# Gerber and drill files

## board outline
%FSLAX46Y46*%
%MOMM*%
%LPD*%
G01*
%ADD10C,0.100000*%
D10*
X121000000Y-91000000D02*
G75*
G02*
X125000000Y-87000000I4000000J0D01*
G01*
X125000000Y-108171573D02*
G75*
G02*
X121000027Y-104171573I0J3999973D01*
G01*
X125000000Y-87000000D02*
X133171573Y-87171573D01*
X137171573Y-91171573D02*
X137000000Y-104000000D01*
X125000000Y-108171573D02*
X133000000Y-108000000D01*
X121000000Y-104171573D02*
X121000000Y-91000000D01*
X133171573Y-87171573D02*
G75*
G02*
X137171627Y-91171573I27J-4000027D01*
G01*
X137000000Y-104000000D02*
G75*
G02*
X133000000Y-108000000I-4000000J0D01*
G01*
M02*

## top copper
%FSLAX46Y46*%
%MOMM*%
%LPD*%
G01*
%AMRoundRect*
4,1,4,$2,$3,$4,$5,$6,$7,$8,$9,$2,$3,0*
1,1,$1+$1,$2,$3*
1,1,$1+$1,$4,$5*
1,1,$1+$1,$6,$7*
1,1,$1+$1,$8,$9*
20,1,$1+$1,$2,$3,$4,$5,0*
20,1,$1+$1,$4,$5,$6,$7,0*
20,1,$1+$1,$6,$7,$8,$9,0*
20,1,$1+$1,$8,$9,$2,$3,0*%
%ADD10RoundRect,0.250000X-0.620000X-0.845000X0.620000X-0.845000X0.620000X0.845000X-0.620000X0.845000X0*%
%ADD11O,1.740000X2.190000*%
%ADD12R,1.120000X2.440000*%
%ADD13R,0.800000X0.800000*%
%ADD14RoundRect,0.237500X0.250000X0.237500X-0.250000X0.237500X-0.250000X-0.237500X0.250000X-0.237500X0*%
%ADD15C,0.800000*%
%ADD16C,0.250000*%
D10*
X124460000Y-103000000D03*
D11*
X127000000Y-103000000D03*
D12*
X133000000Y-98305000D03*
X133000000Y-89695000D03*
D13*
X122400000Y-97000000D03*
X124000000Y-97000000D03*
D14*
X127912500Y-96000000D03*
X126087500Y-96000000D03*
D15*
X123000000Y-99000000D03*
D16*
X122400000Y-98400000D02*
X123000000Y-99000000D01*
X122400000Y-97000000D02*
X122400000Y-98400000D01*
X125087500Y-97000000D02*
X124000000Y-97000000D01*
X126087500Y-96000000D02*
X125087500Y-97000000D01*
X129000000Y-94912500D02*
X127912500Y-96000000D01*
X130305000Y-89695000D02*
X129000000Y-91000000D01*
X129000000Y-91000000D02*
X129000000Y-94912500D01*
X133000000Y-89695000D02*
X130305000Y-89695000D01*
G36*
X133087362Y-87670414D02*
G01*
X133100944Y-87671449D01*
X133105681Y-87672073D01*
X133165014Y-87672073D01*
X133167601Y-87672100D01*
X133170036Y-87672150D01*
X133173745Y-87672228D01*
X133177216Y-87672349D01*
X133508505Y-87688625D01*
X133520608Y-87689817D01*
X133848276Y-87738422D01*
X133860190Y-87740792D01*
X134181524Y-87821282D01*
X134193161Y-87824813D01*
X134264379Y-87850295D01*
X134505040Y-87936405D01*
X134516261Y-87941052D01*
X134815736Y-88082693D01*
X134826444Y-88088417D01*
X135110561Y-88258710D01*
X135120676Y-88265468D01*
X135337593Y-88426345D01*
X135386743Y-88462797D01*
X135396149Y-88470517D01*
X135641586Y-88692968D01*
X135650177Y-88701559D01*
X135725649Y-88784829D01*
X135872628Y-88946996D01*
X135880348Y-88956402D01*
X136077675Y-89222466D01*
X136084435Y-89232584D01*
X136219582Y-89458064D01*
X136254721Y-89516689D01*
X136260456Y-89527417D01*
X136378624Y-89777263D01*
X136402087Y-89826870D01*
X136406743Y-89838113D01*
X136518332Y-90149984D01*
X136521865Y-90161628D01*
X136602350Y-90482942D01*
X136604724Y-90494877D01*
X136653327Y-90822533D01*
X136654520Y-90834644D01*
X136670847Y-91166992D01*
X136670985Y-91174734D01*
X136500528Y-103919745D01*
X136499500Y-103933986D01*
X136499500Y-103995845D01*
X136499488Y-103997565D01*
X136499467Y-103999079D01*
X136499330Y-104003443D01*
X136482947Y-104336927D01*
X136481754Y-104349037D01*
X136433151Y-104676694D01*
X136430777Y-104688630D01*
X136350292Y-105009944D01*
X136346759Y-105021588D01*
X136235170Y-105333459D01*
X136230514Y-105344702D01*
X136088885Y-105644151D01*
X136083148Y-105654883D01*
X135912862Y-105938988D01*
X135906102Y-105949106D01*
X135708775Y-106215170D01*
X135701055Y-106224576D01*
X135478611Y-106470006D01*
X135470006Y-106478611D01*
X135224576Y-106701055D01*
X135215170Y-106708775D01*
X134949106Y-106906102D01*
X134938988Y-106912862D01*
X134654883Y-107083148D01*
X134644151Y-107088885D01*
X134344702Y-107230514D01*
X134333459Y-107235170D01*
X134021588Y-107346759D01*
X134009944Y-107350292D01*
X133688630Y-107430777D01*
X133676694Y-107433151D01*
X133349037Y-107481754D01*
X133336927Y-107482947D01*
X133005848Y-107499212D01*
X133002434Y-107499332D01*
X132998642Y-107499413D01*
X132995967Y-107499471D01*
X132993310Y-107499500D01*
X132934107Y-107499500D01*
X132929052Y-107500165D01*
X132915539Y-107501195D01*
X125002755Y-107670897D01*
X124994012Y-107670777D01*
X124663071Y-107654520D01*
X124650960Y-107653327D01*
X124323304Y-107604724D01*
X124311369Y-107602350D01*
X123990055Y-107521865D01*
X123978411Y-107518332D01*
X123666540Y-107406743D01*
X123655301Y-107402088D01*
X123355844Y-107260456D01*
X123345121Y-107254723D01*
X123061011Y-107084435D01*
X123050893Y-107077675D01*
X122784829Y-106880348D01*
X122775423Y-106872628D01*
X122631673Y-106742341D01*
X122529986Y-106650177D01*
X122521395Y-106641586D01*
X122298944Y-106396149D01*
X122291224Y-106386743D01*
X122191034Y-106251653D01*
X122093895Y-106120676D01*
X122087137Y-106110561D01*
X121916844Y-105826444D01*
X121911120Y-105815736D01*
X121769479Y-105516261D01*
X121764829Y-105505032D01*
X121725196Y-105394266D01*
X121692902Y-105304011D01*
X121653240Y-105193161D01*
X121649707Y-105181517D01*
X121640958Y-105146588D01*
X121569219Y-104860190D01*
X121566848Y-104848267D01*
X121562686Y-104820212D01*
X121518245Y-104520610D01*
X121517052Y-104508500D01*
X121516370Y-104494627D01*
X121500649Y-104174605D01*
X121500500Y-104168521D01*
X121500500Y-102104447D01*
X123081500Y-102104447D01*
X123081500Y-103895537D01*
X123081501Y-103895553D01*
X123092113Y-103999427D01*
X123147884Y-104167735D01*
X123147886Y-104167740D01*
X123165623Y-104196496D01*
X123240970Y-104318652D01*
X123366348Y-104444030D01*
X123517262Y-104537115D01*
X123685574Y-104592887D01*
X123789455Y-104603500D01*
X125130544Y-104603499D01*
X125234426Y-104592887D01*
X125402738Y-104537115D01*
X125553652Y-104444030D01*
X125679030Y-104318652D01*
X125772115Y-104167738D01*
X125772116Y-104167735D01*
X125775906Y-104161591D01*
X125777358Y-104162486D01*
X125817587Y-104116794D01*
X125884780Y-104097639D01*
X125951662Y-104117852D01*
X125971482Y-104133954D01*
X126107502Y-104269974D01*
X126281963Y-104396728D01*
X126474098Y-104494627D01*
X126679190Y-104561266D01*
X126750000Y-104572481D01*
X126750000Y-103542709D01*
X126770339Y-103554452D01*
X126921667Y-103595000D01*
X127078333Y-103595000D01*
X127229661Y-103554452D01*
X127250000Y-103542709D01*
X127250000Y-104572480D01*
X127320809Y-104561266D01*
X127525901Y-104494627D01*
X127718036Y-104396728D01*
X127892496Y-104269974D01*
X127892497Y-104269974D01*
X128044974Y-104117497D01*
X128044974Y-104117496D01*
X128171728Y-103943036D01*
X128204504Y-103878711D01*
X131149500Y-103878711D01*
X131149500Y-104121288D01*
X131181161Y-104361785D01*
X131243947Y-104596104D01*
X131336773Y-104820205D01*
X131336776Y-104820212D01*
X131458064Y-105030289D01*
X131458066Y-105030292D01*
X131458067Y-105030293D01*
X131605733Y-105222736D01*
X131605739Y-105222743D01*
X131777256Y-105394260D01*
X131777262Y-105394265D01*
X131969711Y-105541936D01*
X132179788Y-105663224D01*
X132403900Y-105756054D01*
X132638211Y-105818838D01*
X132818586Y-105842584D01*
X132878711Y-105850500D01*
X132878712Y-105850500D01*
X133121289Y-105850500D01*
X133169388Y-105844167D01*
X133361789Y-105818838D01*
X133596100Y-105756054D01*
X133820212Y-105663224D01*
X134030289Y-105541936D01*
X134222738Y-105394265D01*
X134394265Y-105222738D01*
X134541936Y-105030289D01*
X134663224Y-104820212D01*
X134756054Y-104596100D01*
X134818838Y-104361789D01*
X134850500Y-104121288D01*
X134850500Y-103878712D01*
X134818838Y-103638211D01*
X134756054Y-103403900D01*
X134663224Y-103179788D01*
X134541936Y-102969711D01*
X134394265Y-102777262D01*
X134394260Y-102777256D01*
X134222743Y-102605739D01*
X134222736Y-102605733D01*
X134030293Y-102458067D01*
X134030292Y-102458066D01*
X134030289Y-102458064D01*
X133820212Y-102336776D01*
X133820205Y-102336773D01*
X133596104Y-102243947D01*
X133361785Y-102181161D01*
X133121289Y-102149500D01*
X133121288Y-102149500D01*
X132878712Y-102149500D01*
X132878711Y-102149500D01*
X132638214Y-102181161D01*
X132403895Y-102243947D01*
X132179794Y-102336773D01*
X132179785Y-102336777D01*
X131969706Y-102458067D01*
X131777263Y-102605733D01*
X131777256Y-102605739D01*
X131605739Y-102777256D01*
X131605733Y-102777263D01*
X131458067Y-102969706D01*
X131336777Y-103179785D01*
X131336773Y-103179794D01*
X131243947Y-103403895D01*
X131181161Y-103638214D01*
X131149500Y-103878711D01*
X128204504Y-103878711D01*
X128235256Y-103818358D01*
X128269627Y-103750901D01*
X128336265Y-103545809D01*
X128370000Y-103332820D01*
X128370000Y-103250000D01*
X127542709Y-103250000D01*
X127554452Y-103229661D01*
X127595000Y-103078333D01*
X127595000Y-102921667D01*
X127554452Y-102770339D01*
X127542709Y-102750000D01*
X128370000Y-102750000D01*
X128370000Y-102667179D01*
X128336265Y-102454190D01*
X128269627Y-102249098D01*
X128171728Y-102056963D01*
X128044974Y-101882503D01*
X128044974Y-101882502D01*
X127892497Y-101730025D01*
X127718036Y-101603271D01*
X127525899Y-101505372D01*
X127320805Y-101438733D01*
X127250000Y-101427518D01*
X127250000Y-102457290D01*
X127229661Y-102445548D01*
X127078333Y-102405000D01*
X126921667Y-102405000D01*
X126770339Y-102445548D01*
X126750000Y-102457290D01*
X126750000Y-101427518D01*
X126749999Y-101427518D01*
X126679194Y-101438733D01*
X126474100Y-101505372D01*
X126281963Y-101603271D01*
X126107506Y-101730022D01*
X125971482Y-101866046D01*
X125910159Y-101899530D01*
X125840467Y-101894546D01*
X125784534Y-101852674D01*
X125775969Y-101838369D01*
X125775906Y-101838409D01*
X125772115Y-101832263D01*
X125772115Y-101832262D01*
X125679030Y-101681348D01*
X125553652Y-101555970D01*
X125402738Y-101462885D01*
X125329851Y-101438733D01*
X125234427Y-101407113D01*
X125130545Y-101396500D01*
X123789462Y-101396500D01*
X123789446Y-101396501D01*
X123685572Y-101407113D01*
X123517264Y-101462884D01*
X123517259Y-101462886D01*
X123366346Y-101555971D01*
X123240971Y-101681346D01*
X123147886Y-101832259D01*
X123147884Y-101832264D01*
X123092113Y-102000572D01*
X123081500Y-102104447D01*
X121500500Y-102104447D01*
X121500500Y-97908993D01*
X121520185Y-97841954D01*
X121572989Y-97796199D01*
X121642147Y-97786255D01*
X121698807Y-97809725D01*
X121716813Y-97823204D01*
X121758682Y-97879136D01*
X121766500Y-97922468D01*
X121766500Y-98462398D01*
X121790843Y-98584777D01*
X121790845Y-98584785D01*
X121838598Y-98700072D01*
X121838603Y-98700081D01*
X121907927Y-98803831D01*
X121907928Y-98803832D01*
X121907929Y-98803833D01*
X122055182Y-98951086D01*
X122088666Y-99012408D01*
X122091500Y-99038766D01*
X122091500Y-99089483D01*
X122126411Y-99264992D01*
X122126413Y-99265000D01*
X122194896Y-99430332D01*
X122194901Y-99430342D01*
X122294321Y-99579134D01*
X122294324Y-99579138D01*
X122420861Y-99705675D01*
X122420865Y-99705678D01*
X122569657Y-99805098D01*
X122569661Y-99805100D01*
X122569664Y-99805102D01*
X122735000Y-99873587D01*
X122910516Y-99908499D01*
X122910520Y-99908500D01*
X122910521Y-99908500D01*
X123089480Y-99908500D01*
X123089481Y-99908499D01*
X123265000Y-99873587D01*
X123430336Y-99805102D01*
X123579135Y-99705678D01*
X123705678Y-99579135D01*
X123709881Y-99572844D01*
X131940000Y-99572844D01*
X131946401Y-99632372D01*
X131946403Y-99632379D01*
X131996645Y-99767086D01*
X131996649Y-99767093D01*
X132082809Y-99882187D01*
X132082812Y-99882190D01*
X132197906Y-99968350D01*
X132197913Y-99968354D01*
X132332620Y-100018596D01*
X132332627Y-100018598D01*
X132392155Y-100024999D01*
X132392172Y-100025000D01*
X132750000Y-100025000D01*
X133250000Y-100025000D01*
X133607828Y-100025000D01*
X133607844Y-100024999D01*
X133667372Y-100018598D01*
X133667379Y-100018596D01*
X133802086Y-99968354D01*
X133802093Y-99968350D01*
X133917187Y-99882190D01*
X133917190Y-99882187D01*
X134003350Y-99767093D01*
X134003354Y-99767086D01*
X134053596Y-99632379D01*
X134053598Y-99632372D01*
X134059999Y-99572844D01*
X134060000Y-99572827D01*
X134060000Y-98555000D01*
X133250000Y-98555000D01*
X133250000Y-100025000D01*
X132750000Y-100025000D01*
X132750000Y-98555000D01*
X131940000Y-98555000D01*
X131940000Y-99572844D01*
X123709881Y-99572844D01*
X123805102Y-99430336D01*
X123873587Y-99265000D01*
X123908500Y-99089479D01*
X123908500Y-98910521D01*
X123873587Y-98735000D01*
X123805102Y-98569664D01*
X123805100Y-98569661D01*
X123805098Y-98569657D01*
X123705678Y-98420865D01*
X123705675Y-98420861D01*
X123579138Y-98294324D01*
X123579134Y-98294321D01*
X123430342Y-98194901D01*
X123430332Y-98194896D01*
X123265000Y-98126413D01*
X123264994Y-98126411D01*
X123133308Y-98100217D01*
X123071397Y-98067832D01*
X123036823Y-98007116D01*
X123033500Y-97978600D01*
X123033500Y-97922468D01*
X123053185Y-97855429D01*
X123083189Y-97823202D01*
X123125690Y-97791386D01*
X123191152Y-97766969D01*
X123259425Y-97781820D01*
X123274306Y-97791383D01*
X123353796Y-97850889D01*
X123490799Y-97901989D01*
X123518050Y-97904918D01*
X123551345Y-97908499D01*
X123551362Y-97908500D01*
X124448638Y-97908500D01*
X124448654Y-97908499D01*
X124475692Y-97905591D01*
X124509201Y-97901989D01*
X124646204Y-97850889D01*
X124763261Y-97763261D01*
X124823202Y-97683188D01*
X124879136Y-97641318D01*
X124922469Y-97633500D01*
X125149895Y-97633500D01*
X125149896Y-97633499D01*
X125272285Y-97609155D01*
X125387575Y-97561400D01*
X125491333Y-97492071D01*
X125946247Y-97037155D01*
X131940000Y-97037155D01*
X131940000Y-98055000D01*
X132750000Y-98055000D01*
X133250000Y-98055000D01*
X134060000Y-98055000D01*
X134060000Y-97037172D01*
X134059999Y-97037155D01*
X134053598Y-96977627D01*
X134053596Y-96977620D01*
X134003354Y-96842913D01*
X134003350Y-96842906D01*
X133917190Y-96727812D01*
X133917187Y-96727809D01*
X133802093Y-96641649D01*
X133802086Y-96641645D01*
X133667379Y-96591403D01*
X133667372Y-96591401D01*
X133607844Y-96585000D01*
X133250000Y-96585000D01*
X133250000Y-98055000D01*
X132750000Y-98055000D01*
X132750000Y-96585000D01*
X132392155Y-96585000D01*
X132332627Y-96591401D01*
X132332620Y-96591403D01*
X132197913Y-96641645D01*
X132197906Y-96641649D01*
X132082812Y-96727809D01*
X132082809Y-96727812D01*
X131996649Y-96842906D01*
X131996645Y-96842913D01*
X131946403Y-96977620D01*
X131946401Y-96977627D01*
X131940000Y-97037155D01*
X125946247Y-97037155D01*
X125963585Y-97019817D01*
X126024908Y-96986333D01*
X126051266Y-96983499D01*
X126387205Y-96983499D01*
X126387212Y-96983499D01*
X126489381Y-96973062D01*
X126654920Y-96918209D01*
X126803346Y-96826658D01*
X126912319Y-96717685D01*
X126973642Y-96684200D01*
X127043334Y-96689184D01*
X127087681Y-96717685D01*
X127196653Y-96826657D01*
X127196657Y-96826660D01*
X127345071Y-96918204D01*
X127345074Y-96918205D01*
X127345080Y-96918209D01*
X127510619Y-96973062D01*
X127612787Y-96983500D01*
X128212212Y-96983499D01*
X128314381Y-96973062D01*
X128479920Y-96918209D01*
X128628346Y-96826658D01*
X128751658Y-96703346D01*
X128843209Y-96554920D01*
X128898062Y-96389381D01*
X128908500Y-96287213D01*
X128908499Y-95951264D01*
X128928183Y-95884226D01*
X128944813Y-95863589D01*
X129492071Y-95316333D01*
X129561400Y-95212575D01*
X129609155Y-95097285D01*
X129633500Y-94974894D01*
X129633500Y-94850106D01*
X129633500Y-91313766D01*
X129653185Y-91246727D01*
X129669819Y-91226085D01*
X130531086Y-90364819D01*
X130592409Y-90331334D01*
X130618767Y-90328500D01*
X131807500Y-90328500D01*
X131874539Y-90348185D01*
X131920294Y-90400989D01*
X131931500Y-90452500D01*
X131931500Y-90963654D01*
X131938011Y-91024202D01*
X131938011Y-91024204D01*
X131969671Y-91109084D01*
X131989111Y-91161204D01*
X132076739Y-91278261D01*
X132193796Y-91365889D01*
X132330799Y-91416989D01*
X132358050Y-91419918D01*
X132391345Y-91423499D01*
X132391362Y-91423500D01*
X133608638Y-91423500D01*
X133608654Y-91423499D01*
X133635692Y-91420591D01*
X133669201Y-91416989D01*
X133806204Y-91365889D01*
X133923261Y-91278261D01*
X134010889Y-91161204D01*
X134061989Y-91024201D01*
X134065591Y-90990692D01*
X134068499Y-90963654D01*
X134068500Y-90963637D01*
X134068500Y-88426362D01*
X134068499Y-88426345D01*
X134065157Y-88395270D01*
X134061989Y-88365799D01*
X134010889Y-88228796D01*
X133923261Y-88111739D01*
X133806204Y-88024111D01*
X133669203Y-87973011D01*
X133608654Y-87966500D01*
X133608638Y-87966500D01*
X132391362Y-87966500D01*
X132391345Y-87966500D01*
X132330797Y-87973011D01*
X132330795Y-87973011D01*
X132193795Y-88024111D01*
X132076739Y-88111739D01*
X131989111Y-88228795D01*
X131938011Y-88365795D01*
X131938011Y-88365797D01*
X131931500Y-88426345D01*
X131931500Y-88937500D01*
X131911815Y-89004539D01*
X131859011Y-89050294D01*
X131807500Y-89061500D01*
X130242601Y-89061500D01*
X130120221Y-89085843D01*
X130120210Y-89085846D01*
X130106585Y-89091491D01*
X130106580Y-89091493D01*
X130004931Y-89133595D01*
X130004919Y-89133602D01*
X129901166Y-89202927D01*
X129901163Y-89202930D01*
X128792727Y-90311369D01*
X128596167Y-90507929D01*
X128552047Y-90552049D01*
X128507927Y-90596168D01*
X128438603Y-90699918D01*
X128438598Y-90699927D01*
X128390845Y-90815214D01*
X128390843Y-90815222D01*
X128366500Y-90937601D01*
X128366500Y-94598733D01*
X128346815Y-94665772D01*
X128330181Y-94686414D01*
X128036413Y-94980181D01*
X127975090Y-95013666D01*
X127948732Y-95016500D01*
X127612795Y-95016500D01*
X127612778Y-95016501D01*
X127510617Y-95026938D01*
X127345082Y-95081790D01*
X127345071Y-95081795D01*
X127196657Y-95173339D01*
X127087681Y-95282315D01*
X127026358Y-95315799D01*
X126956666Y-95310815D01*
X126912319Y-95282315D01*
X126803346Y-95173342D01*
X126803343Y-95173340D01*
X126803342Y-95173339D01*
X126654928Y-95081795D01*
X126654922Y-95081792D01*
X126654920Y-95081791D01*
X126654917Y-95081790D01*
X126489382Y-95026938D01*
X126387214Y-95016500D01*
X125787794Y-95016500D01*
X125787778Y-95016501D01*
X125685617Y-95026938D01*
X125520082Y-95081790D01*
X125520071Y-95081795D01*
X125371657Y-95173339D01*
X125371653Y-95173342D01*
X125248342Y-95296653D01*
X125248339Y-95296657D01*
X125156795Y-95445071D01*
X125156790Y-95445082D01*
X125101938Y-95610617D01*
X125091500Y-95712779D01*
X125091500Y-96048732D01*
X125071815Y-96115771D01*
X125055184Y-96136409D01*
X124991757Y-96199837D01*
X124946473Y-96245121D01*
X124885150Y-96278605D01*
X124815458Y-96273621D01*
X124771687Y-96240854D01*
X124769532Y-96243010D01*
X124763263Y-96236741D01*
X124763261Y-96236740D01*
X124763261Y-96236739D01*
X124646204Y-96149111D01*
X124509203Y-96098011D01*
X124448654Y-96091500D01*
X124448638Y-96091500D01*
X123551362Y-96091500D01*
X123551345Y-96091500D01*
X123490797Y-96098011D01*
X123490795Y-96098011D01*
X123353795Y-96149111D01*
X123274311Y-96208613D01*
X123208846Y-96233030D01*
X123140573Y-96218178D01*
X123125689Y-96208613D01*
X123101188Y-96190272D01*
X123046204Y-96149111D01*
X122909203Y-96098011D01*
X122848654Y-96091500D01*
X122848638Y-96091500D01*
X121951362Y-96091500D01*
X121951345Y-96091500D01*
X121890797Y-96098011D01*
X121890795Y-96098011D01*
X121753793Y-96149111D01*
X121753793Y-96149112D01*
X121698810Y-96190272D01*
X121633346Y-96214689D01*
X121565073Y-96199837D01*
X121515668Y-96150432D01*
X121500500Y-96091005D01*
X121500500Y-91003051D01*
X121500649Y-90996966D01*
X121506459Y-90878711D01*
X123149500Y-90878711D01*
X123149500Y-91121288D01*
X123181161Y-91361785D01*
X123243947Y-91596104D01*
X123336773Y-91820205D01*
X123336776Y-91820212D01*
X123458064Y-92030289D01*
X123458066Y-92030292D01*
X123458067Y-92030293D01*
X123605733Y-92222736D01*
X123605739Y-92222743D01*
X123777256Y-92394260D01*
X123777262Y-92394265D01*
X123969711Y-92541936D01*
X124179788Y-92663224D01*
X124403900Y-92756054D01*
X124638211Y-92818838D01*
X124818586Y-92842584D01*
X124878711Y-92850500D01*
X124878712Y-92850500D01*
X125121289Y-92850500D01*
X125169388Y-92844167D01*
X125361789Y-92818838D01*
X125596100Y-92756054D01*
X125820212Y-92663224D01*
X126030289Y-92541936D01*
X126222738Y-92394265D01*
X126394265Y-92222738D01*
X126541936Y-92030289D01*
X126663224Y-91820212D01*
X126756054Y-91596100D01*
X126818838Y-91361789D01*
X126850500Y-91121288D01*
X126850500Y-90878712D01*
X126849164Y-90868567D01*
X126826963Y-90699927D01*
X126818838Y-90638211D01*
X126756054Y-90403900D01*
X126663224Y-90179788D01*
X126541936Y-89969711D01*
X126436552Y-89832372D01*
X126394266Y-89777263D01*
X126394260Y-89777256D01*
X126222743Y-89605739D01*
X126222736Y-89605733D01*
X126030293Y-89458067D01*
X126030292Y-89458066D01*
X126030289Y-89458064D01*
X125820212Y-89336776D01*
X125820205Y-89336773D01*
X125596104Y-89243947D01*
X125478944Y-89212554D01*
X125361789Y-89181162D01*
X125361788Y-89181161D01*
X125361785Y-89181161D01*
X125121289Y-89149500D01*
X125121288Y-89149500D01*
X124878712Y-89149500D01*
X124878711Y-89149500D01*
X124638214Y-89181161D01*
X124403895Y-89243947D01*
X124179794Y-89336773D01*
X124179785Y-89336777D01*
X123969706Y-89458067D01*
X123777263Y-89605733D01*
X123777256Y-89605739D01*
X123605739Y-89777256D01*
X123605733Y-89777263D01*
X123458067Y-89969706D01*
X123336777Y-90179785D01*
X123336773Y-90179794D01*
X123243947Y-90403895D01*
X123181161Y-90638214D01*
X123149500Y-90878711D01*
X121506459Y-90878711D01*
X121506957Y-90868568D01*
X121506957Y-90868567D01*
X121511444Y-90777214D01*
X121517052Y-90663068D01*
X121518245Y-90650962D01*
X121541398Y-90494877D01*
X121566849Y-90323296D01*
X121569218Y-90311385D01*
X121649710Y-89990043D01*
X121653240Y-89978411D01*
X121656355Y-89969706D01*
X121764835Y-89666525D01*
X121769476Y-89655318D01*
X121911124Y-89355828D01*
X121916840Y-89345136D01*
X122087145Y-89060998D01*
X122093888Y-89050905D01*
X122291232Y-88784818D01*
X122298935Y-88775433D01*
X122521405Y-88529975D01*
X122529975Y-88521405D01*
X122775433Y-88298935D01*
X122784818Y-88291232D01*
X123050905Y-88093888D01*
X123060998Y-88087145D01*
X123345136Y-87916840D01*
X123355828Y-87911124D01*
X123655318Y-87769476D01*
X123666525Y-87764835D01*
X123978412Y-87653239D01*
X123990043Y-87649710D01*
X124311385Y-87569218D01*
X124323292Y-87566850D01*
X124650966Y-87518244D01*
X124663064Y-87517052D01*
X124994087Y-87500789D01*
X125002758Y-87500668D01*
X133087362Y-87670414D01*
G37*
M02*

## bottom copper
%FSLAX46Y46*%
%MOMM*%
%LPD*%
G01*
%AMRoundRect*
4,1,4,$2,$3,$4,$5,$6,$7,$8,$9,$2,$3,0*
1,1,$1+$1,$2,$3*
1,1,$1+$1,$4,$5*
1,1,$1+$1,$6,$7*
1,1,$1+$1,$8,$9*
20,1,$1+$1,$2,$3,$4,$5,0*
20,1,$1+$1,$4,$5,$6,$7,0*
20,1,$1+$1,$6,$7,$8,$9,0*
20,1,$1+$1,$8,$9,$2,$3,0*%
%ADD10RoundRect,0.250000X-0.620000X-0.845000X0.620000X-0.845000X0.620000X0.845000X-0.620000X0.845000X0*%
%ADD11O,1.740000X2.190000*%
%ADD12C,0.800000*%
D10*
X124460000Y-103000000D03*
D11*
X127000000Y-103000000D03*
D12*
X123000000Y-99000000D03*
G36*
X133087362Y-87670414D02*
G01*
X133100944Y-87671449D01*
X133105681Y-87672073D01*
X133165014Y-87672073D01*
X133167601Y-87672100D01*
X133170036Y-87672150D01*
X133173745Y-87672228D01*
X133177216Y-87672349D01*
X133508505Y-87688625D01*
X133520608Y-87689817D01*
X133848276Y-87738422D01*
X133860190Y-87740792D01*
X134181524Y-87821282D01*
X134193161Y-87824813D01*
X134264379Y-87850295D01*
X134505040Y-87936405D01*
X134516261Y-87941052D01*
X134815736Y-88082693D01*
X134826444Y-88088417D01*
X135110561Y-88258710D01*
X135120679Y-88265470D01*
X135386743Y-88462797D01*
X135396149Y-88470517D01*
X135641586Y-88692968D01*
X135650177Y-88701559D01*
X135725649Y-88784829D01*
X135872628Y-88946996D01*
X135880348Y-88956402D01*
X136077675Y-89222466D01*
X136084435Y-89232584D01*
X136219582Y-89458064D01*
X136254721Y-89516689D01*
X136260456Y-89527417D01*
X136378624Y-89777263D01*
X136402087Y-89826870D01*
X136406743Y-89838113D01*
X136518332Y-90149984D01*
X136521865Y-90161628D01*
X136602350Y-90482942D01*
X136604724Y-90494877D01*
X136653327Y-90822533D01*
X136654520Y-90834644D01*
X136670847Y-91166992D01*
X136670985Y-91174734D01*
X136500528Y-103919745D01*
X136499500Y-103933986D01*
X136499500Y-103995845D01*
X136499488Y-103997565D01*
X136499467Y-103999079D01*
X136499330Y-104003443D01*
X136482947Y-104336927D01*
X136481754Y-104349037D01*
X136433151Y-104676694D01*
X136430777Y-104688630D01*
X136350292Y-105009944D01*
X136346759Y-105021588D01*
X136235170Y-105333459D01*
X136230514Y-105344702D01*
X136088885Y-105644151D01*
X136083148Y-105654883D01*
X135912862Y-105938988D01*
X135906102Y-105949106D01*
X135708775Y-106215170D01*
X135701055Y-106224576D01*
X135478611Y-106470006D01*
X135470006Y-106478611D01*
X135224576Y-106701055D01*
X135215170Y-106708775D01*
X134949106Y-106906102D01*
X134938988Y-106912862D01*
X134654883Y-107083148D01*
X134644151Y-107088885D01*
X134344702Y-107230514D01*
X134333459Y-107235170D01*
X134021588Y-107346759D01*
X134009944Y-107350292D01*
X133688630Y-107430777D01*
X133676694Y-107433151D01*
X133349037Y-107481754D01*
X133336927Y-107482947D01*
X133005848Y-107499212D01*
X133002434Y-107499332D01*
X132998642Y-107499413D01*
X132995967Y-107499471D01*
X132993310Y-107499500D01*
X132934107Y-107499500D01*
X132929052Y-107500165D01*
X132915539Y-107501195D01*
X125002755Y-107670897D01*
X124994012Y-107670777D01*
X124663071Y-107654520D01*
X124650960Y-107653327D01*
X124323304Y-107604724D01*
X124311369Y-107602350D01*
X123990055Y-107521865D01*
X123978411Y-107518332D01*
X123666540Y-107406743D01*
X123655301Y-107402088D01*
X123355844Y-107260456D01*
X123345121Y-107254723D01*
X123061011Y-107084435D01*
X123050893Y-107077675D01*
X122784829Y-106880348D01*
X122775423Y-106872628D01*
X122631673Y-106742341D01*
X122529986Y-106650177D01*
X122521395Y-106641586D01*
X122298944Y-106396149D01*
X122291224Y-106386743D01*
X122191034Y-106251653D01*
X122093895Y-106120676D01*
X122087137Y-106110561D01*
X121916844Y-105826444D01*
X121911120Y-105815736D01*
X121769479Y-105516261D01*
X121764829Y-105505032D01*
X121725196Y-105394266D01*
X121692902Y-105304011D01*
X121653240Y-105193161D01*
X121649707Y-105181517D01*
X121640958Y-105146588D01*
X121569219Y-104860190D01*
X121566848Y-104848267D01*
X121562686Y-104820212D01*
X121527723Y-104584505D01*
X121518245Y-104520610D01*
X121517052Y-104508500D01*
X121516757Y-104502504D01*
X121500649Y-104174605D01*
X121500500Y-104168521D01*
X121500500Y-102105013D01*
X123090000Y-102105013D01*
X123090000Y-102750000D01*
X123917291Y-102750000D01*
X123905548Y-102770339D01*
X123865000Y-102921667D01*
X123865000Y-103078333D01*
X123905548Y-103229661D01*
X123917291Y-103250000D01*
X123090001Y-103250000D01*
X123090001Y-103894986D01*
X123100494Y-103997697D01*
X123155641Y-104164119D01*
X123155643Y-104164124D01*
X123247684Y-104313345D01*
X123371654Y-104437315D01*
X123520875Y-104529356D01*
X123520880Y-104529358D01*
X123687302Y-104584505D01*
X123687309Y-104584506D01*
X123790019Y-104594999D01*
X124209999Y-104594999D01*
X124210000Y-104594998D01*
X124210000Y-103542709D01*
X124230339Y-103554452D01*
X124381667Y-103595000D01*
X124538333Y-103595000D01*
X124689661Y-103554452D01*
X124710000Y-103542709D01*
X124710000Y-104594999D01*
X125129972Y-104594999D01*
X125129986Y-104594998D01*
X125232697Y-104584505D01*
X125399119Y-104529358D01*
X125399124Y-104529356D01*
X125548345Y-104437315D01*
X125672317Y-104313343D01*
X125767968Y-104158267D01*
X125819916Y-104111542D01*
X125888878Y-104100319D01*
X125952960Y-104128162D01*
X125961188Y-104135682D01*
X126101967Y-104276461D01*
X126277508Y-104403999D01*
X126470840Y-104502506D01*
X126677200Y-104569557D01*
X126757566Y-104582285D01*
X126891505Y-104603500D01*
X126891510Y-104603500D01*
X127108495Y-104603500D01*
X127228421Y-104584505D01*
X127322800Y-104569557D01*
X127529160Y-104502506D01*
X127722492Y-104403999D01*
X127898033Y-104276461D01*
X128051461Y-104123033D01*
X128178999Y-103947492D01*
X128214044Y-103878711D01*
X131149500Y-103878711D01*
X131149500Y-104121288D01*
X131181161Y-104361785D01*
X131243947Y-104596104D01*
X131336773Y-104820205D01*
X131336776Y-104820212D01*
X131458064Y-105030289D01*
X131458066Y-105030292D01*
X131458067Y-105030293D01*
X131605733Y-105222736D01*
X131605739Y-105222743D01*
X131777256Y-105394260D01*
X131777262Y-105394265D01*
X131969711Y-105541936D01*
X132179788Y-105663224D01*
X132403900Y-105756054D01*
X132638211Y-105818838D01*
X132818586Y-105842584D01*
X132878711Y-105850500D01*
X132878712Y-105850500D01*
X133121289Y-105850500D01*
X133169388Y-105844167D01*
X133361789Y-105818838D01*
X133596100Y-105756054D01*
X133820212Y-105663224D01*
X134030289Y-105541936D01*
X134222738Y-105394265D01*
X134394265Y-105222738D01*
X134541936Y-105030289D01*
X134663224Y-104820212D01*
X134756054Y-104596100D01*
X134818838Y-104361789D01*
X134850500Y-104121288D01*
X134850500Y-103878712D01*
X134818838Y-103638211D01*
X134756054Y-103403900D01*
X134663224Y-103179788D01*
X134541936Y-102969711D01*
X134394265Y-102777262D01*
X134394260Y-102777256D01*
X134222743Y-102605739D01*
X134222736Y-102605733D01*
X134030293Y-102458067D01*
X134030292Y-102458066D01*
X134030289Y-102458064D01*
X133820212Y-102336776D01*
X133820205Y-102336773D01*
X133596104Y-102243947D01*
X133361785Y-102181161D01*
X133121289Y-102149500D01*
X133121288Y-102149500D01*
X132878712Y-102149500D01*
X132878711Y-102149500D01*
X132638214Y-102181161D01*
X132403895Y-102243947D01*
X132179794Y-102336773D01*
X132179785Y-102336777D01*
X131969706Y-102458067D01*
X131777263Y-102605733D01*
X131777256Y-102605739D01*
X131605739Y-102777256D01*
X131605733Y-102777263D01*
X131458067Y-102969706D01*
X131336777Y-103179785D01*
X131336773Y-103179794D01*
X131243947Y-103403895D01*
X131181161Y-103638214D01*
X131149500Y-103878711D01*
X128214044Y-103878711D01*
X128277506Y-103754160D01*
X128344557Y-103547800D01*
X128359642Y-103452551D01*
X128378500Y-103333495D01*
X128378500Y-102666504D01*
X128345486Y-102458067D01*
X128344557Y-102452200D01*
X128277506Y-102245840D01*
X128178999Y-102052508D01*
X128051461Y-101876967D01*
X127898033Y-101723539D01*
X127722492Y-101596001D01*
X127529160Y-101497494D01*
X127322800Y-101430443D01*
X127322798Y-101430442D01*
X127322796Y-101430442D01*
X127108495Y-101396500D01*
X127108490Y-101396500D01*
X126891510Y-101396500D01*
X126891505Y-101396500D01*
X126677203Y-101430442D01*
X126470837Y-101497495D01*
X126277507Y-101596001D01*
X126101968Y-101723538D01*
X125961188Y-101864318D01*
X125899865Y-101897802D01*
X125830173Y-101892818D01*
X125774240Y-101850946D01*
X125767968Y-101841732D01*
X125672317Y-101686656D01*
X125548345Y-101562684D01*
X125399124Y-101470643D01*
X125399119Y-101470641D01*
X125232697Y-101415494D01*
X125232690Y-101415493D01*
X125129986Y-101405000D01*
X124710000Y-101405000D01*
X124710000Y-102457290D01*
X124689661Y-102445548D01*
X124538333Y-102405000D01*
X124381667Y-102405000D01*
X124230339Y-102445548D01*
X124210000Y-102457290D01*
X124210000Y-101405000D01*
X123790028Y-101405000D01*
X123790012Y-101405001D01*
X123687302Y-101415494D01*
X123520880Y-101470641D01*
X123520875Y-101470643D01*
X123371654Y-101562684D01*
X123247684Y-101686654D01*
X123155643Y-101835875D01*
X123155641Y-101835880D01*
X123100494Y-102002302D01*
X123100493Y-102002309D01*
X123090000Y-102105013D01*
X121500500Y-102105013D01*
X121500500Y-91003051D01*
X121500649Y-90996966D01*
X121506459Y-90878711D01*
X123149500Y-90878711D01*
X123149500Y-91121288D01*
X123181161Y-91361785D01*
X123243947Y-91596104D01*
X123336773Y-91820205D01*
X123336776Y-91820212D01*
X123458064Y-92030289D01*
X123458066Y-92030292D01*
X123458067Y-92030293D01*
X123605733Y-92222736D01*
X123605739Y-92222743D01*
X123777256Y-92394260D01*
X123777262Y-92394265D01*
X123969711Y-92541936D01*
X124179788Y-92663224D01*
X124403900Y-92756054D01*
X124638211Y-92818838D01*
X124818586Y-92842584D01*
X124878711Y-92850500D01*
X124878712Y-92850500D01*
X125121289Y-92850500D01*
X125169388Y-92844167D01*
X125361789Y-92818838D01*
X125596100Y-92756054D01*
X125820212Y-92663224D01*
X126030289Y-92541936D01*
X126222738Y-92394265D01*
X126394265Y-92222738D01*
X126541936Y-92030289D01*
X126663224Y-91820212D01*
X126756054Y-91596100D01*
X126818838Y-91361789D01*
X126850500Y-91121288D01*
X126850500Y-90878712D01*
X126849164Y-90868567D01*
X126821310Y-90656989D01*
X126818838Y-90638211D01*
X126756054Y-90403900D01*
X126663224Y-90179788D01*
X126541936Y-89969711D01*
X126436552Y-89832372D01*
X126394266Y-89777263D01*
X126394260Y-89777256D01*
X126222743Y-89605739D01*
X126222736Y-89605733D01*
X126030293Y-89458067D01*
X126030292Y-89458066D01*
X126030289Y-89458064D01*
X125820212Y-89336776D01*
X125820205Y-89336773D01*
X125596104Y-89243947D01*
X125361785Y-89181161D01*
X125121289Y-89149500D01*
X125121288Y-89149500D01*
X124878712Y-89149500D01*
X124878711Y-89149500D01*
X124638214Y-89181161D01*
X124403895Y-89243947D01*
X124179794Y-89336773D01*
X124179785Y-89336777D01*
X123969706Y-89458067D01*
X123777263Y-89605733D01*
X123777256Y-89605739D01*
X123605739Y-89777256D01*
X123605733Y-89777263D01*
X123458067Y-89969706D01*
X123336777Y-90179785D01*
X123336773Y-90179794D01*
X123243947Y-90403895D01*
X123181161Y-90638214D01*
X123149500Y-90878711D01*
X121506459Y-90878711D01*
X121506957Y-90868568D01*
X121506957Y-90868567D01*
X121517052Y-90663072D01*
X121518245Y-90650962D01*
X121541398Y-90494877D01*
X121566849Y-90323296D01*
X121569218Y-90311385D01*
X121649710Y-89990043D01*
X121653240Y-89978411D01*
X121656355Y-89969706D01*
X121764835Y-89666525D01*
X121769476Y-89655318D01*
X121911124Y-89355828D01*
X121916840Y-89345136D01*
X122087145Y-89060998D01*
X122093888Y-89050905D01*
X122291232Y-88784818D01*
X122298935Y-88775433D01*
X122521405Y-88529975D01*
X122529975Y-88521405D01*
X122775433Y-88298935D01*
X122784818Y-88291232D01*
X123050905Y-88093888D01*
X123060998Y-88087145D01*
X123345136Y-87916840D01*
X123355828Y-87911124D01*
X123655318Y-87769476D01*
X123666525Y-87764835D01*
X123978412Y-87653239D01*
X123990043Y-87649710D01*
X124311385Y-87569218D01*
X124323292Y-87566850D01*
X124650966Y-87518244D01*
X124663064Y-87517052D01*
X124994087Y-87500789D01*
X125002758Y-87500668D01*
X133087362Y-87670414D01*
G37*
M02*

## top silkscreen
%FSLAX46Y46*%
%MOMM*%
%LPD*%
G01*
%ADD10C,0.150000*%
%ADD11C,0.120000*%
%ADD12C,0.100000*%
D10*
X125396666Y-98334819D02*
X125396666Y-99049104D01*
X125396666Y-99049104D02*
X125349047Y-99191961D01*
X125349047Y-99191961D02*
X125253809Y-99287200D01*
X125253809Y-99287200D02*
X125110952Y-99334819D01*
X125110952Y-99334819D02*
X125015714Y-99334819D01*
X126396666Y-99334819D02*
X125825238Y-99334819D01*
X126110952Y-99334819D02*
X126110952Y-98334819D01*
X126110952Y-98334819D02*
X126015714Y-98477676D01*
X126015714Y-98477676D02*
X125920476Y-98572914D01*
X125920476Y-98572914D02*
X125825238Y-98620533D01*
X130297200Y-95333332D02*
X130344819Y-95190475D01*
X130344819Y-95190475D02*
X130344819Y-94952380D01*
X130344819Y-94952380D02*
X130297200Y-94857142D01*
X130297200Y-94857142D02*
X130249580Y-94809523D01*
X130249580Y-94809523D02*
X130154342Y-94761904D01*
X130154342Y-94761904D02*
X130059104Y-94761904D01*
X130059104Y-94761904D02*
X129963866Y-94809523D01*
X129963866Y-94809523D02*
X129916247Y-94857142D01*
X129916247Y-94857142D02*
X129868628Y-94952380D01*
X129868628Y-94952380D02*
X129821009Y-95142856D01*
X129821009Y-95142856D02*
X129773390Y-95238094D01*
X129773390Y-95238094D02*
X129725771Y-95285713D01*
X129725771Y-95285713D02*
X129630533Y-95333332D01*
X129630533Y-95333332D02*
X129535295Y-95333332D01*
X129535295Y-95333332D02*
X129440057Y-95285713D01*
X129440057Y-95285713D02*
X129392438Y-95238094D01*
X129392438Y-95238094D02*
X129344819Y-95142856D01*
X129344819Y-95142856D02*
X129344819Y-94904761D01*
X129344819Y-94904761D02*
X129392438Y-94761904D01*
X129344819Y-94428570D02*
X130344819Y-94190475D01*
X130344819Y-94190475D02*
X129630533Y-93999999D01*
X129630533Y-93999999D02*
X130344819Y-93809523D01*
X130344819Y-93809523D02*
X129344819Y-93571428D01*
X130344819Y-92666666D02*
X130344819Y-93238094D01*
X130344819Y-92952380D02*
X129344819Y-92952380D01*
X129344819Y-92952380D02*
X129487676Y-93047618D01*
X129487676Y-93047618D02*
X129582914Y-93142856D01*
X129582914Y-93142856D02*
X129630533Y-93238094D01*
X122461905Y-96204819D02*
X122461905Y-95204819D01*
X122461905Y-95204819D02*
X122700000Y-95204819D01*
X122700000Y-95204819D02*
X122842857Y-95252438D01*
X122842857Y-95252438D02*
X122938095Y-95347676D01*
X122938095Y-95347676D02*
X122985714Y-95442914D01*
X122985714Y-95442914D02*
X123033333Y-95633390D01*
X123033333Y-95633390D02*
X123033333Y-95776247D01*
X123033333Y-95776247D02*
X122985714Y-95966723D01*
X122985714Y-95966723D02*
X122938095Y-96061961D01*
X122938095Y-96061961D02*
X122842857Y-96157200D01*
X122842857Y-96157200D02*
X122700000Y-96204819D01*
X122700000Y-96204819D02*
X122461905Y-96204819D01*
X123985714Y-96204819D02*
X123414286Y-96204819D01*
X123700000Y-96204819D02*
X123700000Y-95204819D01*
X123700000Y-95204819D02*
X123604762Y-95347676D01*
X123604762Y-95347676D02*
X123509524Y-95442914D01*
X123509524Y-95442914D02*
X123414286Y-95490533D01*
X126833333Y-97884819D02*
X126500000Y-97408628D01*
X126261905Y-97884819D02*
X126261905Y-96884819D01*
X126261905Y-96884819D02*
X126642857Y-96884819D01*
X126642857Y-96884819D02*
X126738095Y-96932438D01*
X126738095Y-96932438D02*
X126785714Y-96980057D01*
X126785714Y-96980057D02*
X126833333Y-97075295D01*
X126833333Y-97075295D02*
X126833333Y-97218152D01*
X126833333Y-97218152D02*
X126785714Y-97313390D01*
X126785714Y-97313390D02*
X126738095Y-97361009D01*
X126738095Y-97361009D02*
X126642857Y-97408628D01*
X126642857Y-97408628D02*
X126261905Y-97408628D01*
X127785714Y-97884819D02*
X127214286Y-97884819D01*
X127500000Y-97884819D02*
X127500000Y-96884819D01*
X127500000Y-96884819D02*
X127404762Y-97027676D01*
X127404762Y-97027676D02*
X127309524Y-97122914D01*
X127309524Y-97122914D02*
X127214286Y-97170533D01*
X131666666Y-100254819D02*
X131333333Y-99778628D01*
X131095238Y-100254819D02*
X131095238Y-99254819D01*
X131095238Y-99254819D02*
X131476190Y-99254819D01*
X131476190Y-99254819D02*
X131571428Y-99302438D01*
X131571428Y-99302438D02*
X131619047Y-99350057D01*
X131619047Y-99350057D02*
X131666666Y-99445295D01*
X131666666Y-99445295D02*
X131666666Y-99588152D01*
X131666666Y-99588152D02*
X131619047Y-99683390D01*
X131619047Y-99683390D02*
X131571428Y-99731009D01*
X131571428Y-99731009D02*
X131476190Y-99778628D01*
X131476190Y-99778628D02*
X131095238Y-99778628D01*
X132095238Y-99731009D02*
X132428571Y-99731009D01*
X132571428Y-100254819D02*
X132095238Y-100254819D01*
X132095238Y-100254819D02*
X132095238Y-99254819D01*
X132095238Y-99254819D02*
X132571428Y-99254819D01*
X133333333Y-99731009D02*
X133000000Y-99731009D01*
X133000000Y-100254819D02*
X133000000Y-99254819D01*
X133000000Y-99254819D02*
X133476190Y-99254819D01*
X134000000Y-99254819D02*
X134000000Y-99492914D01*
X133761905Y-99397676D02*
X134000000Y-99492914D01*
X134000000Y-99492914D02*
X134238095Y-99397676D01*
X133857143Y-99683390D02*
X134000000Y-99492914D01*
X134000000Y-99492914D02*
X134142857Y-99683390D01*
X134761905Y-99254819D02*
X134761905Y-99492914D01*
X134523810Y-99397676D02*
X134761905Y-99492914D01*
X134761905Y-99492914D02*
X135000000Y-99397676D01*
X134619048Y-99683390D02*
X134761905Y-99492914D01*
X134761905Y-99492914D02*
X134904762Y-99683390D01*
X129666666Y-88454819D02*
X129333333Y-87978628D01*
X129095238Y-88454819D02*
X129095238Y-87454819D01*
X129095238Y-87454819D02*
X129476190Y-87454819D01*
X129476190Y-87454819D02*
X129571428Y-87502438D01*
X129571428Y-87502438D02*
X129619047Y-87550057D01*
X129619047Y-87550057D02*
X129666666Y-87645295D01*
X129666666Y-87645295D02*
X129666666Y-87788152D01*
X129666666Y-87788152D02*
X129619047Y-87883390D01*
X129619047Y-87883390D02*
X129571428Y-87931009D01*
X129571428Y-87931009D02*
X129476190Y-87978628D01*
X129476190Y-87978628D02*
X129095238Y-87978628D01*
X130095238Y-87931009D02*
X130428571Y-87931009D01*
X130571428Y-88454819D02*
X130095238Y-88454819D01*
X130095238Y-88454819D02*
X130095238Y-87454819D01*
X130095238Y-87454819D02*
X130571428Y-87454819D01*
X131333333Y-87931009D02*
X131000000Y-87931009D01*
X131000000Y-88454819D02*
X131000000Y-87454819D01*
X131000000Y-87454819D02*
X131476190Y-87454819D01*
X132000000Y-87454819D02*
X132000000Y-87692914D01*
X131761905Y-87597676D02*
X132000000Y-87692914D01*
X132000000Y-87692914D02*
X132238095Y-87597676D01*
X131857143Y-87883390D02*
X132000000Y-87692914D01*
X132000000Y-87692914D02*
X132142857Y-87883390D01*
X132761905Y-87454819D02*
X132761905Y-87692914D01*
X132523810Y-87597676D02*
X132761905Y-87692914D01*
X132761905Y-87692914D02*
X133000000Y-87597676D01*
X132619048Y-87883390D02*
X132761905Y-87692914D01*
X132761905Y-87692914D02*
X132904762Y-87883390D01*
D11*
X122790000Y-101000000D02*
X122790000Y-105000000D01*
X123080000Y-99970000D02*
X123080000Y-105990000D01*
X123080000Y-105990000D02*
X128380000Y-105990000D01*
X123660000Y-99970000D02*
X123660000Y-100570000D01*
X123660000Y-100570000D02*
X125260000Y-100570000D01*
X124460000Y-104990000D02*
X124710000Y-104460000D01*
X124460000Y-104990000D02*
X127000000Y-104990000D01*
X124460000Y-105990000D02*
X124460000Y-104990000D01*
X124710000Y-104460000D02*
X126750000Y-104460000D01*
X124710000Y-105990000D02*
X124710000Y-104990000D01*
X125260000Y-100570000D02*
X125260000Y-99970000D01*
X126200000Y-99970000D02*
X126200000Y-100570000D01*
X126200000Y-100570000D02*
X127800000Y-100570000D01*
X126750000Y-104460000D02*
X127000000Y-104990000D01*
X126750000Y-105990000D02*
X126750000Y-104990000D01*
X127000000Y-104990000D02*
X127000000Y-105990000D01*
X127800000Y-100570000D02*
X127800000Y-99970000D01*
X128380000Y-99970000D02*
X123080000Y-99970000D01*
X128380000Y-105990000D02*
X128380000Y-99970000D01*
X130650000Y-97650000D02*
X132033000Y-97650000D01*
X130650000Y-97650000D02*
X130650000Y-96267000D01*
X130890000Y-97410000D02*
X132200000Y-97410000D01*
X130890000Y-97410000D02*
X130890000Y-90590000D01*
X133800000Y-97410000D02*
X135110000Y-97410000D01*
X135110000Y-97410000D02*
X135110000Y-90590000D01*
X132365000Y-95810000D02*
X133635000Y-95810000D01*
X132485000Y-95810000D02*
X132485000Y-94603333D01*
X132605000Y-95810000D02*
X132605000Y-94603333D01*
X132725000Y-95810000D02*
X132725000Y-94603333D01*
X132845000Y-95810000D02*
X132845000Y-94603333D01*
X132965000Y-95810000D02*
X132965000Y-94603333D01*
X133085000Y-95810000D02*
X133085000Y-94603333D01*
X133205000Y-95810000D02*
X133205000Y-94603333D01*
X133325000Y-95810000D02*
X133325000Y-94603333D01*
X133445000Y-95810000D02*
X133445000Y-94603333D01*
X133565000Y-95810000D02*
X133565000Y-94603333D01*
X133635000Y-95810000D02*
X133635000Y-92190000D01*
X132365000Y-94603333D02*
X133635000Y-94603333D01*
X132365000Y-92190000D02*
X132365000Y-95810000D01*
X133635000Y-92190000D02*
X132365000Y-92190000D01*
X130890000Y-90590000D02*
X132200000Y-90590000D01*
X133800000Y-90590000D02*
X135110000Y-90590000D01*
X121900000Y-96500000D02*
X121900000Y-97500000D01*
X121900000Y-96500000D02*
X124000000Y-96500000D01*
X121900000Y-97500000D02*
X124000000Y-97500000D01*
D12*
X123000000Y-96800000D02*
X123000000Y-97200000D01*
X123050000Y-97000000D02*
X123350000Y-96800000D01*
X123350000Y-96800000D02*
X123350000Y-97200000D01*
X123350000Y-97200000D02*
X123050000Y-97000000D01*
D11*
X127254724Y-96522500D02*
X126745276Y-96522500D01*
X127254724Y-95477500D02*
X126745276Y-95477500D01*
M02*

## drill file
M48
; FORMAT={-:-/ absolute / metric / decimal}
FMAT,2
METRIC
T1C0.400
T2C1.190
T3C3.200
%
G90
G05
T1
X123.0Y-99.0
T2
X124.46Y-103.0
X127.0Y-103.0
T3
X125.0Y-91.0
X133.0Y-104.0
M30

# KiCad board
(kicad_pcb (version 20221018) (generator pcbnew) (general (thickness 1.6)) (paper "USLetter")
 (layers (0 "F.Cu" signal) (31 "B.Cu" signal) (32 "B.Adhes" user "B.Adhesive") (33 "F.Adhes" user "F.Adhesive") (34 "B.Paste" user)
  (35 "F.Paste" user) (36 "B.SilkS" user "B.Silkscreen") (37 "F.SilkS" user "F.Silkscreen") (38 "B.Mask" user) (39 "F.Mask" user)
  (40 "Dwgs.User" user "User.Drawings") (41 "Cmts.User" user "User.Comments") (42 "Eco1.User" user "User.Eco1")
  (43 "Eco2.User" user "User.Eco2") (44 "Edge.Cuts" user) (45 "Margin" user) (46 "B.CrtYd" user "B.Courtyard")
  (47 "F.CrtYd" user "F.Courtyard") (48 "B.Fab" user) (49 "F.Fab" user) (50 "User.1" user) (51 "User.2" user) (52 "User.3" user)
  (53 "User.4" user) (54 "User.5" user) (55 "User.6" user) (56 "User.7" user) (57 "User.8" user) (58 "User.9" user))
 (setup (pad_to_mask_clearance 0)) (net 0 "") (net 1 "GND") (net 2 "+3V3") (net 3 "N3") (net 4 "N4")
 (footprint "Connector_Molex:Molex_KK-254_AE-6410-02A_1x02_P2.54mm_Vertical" (layer "F.Cu") (at 124.46 103)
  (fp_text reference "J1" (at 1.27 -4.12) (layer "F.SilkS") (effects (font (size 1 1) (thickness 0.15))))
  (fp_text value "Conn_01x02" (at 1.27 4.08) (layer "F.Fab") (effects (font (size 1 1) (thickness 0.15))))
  (fp_line (start -1.67 -2) (end -1.67 2) (stroke (width 0.12) (type solid)) (layer "F.SilkS"))
  (fp_line (start -1.38 -3.03) (end -1.38 2.99) (stroke (width 0.12) (type solid)) (layer "F.SilkS"))
  (fp_line (start -1.38 2.99) (end 3.92 2.99) (stroke (width 0.12) (type solid)) (layer "F.SilkS"))
  (fp_line (start -0.8 -3.03) (end -0.8 -2.43) (stroke (width 0.12) (type solid)) (layer "F.SilkS"))
  (fp_line (start -0.8 -2.43) (end 0.8 -2.43) (stroke (width 0.12) (type solid)) (layer "F.SilkS"))
  (fp_line (start 0 1.99) (end 0.25 1.46) (stroke (width 0.12) (type solid)) (layer "F.SilkS"))
  (fp_line (start 0 1.99) (end 2.54 1.99) (stroke (width 0.12) (type solid)) (layer "F.SilkS"))
  (fp_line (start 0 2.99) (end 0 1.99) (stroke (width 0.12) (type solid)) (layer "F.SilkS"))
  (fp_line (start 0.25 1.46) (end 2.29 1.46) (stroke (width 0.12) (type solid)) (layer "F.SilkS"))
  (fp_line (start 0.25 2.99) (end 0.25 1.99) (stroke (width 0.12) (type solid)) (layer "F.SilkS"))
  (fp_line (start 0.8 -2.43) (end 0.8 -3.03) (stroke (width 0.12) (type solid)) (layer "F.SilkS"))
  (fp_line (start 1.74 -3.03) (end 1.74 -2.43) (stroke (width 0.12) (type solid)) (layer "F.SilkS"))
  (fp_line (start 1.74 -2.43) (end 3.34 -2.43) (stroke (width 0.12) (type solid)) (layer "F.SilkS"))
  (fp_line (start 2.29 1.46) (end 2.54 1.99) (stroke (width 0.12) (type solid)) (layer "F.SilkS"))
  (fp_line (start 2.29 2.99) (end 2.29 1.99) (stroke (width 0.12) (type solid)) (layer "F.SilkS"))
  (fp_line (start 2.54 1.99) (end 2.54 2.99) (stroke (width 0.12) (type solid)) (layer "F.SilkS"))
  (fp_line (start 3.34 -2.43) (end 3.34 -3.03) (stroke (width 0.12) (type solid)) (layer "F.SilkS"))
  (fp_line (start 3.92 -3.03) (end -1.38 -3.03) (stroke (width 0.12) (type solid)) (layer "F.SilkS"))
  (fp_line (start 3.92 2.99) (end 3.92 -3.03) (stroke (width 0.12) (type solid)) (layer "F.SilkS"))
  (pad "1" thru_hole roundrect (at 0 0) (size 1.74 2.19) (drill 1.19) (layers "*.Cu" "*.Mask") (roundrect_rratio 0.143678) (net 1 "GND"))
  (pad "2" thru_hole oval (at 2.54 0) (size 1.74 2.19) (drill 1.19) (layers "*.Cu" "*.Mask") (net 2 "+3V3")))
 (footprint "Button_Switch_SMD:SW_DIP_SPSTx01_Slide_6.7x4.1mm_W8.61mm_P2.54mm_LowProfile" (layer "F.Cu") (at 133 94 90)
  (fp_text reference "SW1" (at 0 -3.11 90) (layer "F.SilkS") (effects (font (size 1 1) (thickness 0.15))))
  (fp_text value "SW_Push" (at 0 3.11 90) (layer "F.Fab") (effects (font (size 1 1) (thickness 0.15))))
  (fp_line (start -3.65 -2.35) (end -3.65 -0.967) (stroke (width 0.12) (type solid)) (layer "F.SilkS"))
  (fp_line (start -3.65 -2.35) (end -2.267 -2.35) (stroke (width 0.12) (type solid)) (layer "F.SilkS"))
  (fp_line (start -3.41 -2.11) (end -3.41 -0.8) (stroke (width 0.12) (type solid)) (layer "F.SilkS"))
  (fp_line (start -3.41 -2.11) (end 3.41 -2.11) (stroke (width 0.12) (type solid)) (layer "F.SilkS"))
  (fp_line (start -3.41 0.8) (end -3.41 2.11) (stroke (width 0.12) (type solid)) (layer "F.SilkS"))
  (fp_line (start -3.41 2.11) (end 3.41 2.11) (stroke (width 0.12) (type solid)) (layer "F.SilkS"))
  (fp_line (start -1.81 -0.635) (end -1.81 0.635) (stroke (width 0.12) (type solid)) (layer "F.SilkS"))
  (fp_line (start -1.81 -0.515) (end -0.603333 -0.515) (stroke (width 0.12) (type solid)) (layer "F.SilkS"))
  (fp_line (start -1.81 -0.395) (end -0.603333 -0.395) (stroke (width 0.12) (type solid)) (layer "F.SilkS"))
  (fp_line (start -1.81 -0.275) (end -0.603333 -0.275) (stroke (width 0.12) (type solid)) (layer "F.SilkS"))
  (fp_line (start -1.81 -0.155) (end -0.603333 -0.155) (stroke (width 0.12) (type solid)) (layer "F.SilkS"))
  (fp_line (start -1.81 -0.035) (end -0.603333 -0.035) (stroke (width 0.12) (type solid)) (layer "F.SilkS"))
  (fp_line (start -1.81 0.085) (end -0.603333 0.085) (stroke (width 0.12) (type solid)) (layer "F.SilkS"))
  (fp_line (start -1.81 0.205) (end -0.603333 0.205) (stroke (width 0.12) (type solid)) (layer "F.SilkS"))
  (fp_line (start -1.81 0.325) (end -0.603333 0.325) (stroke (width 0.12) (type solid)) (layer "F.SilkS"))
  (fp_line (start -1.81 0.445) (end -0.603333 0.445) (stroke (width 0.12) (type solid)) (layer "F.SilkS"))
  (fp_line (start -1.81 0.565) (end -0.603333 0.565) (stroke (width 0.12) (type solid)) (layer "F.SilkS"))
  (fp_line (start -1.81 0.635) (end 1.81 0.635) (stroke (width 0.12) (type solid)) (layer "F.SilkS"))
  (fp_line (start -0.603333 -0.635) (end -0.603333 0.635) (stroke (width 0.12) (type solid)) (layer "F.SilkS"))
  (fp_line (start 1.81 -0.635) (end -1.81 -0.635) (stroke (width 0.12) (type solid)) (layer "F.SilkS"))
  (fp_line (start 1.81 0.635) (end 1.81 -0.635) (stroke (width 0.12) (type solid)) (layer "F.SilkS"))
  (fp_line (start 3.41 -2.11) (end 3.41 -0.8) (stroke (width 0.12) (type solid)) (layer "F.SilkS"))
  (fp_line (start 3.41 0.8) (end 3.41 2.11) (stroke (width 0.12) (type solid)) (layer "F.SilkS"))
  (pad "1" smd rect (at -4.305 0 90) (size 2.44 1.12) (layers "F.Cu" "F.Paste" "F.Mask") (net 2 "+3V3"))
  (pad "2" smd rect (at 4.305 0 90) (size 2.44 1.12) (layers "F.Cu" "F.Paste" "F.Mask") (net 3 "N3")))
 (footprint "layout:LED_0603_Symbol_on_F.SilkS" (layer "F.Cu") (at 123.2 97)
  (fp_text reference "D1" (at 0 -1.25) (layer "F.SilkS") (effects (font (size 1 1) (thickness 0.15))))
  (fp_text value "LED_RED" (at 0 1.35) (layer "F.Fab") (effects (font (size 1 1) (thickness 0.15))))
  (fp_line (start -1.3 -0.5) (end -1.3 0.5) (stroke (width 0.12) (type solid)) (layer "F.SilkS"))
  (fp_line (start -1.3 -0.5) (end 0.8 -0.5) (stroke (width 0.12) (type solid)) (layer "F.SilkS"))
  (fp_line (start -1.3 0.5) (end 0.8 0.5) (stroke (width 0.12) (type solid)) (layer "F.SilkS"))
  (fp_line (start -0.2 -0.2) (end -0.2 0.2) (stroke (width 0.1) (type solid)) (layer "F.SilkS"))
  (fp_line (start -0.15 0) (end 0.15 -0.2) (stroke (width 0.1) (type solid)) (layer "F.SilkS"))
  (fp_line (start 0.15 -0.2) (end 0.15 0.2) (stroke (width 0.1) (type solid)) (layer "F.SilkS"))
  (fp_line (start 0.15 0.2) (end -0.15 0) (stroke (width 0.1) (type solid)) (layer "F.SilkS"))
  (pad "1" smd rect (at -0.8 0 180) (size 0.8 0.8) (layers "F.Cu" "F.Paste" "F.Mask") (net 1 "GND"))
  (pad "2" smd rect (at 0.8 0 180) (size 0.8 0.8) (layers "F.Cu" "F.Paste" "F.Mask") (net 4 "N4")))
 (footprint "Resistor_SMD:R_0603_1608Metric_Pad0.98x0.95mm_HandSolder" (layer "F.Cu") (at 127 96 180)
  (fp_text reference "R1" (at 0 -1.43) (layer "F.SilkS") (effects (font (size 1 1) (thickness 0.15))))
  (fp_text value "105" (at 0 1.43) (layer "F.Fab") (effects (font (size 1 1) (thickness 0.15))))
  (fp_line (start -0.254724 -0.5225) (end 0.254724 -0.5225) (stroke (width 0.12) (type solid)) (layer "F.SilkS"))
  (fp_line (start -0.254724 0.5225) (end 0.254724 0.5225) (stroke (width 0.12) (type solid)) (layer "F.SilkS"))
  (pad "1" smd roundrect (at -0.9125 0 180) (size 0.975 0.95) (layers "F.Cu" "F.Paste" "F.Mask") (roundrect_rratio 0.25) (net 3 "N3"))
  (pad "2" smd roundrect (at 0.9125 0 180) (size 0.975 0.95) (layers "F.Cu" "F.Paste" "F.Mask") (roundrect_rratio 0.25) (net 4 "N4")))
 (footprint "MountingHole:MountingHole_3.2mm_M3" (layer "F.Cu") (at 133 104)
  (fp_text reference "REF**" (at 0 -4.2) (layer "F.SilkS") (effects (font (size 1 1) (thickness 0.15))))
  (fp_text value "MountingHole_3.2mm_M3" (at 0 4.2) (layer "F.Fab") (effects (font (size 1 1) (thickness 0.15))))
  (pad "" np_thru_hole circle (at 0 0) (size 3.2 3.2) (drill 3.2) (layers "*.Cu" "*.Mask")))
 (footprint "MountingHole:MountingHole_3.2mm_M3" (layer "F.Cu") (at 125 91)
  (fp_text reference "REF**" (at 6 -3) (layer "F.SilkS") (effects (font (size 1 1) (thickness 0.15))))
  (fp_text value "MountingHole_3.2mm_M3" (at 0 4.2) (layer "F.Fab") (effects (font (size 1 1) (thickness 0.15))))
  (pad "" np_thru_hole circle (at 0 0) (size 3.2 3.2) (drill 3.2) (layers "*.Cu" "*.Mask")))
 (gr_arc (start 121 91) (mid 122.171573 88.171573) (end 125 87) (stroke (width 0.1) (type default)) (layer "Edge.Cuts"))
 (gr_arc (start 125 108.171573) (mid 122.171573 107) (end 121 104.171573) (stroke (width 0.1) (type default)) (layer "Edge.Cuts"))
 (gr_line (start 125 87) (end 133.171573 87.171573) (stroke (width 0.1) (type default)) (layer "Edge.Cuts"))
 (gr_line (start 137.171573 91.171573) (end 137 104) (stroke (width 0.1) (type default)) (layer "Edge.Cuts"))
 (gr_line (start 125 108.171573) (end 133 108) (stroke (width 0.1) (type default)) (layer "Edge.Cuts"))
 (gr_line (start 121 104.171573) (end 121 91) (stroke (width 0.1) (type default)) (layer "Edge.Cuts"))
 (gr_arc (start 133.171573 87.171573) (mid 136 88.343146) (end 137.171573 91.171573) (stroke (width 0.1) (type default)) (layer "Edge.Cuts"))
 (gr_arc (start 137 104) (mid 135.828427 106.828427) (end 133 108) (stroke (width 0.1) (type default)) (layer "Edge.Cuts"))
 (segment (start 122.4 98.4) (end 123 99) (width 0.25) (layer "F.Cu") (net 1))
 (segment (start 122.4 97) (end 122.4 98.4) (width 0.25) (layer "F.Cu") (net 1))
 (via (at 123 99) (size 0.8) (drill 0.4) (layers "F.Cu" "B.Cu") (free) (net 1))
 (segment (start 125.0875 97) (end 124 97) (width 0.25) (layer "F.Cu") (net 4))
 (segment (start 126.0875 96) (end 125.0875 97) (width 0.25) (layer "F.Cu") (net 4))
 (segment (start 129 94.9125) (end 127.9125 96) (width 0.25) (layer "F.Cu") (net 3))
 (segment (start 130.305 89.695) (end 129 91) (width 0.25) (layer "F.Cu") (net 3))
 (segment (start 129 91) (end 129 94.9125) (width 0.25) (layer "F.Cu") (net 3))
 (segment (start 133 89.695) (end 130.305 89.695) (width 0.25) (layer "F.Cu") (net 3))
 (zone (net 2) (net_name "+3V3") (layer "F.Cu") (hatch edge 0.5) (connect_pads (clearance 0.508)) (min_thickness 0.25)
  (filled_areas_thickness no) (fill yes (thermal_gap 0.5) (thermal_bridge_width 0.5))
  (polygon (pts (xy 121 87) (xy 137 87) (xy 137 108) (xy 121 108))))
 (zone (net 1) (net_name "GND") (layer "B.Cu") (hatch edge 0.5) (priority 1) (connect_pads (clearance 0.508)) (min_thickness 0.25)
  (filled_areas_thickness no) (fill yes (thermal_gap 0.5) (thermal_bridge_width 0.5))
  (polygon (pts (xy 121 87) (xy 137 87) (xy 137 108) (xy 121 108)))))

